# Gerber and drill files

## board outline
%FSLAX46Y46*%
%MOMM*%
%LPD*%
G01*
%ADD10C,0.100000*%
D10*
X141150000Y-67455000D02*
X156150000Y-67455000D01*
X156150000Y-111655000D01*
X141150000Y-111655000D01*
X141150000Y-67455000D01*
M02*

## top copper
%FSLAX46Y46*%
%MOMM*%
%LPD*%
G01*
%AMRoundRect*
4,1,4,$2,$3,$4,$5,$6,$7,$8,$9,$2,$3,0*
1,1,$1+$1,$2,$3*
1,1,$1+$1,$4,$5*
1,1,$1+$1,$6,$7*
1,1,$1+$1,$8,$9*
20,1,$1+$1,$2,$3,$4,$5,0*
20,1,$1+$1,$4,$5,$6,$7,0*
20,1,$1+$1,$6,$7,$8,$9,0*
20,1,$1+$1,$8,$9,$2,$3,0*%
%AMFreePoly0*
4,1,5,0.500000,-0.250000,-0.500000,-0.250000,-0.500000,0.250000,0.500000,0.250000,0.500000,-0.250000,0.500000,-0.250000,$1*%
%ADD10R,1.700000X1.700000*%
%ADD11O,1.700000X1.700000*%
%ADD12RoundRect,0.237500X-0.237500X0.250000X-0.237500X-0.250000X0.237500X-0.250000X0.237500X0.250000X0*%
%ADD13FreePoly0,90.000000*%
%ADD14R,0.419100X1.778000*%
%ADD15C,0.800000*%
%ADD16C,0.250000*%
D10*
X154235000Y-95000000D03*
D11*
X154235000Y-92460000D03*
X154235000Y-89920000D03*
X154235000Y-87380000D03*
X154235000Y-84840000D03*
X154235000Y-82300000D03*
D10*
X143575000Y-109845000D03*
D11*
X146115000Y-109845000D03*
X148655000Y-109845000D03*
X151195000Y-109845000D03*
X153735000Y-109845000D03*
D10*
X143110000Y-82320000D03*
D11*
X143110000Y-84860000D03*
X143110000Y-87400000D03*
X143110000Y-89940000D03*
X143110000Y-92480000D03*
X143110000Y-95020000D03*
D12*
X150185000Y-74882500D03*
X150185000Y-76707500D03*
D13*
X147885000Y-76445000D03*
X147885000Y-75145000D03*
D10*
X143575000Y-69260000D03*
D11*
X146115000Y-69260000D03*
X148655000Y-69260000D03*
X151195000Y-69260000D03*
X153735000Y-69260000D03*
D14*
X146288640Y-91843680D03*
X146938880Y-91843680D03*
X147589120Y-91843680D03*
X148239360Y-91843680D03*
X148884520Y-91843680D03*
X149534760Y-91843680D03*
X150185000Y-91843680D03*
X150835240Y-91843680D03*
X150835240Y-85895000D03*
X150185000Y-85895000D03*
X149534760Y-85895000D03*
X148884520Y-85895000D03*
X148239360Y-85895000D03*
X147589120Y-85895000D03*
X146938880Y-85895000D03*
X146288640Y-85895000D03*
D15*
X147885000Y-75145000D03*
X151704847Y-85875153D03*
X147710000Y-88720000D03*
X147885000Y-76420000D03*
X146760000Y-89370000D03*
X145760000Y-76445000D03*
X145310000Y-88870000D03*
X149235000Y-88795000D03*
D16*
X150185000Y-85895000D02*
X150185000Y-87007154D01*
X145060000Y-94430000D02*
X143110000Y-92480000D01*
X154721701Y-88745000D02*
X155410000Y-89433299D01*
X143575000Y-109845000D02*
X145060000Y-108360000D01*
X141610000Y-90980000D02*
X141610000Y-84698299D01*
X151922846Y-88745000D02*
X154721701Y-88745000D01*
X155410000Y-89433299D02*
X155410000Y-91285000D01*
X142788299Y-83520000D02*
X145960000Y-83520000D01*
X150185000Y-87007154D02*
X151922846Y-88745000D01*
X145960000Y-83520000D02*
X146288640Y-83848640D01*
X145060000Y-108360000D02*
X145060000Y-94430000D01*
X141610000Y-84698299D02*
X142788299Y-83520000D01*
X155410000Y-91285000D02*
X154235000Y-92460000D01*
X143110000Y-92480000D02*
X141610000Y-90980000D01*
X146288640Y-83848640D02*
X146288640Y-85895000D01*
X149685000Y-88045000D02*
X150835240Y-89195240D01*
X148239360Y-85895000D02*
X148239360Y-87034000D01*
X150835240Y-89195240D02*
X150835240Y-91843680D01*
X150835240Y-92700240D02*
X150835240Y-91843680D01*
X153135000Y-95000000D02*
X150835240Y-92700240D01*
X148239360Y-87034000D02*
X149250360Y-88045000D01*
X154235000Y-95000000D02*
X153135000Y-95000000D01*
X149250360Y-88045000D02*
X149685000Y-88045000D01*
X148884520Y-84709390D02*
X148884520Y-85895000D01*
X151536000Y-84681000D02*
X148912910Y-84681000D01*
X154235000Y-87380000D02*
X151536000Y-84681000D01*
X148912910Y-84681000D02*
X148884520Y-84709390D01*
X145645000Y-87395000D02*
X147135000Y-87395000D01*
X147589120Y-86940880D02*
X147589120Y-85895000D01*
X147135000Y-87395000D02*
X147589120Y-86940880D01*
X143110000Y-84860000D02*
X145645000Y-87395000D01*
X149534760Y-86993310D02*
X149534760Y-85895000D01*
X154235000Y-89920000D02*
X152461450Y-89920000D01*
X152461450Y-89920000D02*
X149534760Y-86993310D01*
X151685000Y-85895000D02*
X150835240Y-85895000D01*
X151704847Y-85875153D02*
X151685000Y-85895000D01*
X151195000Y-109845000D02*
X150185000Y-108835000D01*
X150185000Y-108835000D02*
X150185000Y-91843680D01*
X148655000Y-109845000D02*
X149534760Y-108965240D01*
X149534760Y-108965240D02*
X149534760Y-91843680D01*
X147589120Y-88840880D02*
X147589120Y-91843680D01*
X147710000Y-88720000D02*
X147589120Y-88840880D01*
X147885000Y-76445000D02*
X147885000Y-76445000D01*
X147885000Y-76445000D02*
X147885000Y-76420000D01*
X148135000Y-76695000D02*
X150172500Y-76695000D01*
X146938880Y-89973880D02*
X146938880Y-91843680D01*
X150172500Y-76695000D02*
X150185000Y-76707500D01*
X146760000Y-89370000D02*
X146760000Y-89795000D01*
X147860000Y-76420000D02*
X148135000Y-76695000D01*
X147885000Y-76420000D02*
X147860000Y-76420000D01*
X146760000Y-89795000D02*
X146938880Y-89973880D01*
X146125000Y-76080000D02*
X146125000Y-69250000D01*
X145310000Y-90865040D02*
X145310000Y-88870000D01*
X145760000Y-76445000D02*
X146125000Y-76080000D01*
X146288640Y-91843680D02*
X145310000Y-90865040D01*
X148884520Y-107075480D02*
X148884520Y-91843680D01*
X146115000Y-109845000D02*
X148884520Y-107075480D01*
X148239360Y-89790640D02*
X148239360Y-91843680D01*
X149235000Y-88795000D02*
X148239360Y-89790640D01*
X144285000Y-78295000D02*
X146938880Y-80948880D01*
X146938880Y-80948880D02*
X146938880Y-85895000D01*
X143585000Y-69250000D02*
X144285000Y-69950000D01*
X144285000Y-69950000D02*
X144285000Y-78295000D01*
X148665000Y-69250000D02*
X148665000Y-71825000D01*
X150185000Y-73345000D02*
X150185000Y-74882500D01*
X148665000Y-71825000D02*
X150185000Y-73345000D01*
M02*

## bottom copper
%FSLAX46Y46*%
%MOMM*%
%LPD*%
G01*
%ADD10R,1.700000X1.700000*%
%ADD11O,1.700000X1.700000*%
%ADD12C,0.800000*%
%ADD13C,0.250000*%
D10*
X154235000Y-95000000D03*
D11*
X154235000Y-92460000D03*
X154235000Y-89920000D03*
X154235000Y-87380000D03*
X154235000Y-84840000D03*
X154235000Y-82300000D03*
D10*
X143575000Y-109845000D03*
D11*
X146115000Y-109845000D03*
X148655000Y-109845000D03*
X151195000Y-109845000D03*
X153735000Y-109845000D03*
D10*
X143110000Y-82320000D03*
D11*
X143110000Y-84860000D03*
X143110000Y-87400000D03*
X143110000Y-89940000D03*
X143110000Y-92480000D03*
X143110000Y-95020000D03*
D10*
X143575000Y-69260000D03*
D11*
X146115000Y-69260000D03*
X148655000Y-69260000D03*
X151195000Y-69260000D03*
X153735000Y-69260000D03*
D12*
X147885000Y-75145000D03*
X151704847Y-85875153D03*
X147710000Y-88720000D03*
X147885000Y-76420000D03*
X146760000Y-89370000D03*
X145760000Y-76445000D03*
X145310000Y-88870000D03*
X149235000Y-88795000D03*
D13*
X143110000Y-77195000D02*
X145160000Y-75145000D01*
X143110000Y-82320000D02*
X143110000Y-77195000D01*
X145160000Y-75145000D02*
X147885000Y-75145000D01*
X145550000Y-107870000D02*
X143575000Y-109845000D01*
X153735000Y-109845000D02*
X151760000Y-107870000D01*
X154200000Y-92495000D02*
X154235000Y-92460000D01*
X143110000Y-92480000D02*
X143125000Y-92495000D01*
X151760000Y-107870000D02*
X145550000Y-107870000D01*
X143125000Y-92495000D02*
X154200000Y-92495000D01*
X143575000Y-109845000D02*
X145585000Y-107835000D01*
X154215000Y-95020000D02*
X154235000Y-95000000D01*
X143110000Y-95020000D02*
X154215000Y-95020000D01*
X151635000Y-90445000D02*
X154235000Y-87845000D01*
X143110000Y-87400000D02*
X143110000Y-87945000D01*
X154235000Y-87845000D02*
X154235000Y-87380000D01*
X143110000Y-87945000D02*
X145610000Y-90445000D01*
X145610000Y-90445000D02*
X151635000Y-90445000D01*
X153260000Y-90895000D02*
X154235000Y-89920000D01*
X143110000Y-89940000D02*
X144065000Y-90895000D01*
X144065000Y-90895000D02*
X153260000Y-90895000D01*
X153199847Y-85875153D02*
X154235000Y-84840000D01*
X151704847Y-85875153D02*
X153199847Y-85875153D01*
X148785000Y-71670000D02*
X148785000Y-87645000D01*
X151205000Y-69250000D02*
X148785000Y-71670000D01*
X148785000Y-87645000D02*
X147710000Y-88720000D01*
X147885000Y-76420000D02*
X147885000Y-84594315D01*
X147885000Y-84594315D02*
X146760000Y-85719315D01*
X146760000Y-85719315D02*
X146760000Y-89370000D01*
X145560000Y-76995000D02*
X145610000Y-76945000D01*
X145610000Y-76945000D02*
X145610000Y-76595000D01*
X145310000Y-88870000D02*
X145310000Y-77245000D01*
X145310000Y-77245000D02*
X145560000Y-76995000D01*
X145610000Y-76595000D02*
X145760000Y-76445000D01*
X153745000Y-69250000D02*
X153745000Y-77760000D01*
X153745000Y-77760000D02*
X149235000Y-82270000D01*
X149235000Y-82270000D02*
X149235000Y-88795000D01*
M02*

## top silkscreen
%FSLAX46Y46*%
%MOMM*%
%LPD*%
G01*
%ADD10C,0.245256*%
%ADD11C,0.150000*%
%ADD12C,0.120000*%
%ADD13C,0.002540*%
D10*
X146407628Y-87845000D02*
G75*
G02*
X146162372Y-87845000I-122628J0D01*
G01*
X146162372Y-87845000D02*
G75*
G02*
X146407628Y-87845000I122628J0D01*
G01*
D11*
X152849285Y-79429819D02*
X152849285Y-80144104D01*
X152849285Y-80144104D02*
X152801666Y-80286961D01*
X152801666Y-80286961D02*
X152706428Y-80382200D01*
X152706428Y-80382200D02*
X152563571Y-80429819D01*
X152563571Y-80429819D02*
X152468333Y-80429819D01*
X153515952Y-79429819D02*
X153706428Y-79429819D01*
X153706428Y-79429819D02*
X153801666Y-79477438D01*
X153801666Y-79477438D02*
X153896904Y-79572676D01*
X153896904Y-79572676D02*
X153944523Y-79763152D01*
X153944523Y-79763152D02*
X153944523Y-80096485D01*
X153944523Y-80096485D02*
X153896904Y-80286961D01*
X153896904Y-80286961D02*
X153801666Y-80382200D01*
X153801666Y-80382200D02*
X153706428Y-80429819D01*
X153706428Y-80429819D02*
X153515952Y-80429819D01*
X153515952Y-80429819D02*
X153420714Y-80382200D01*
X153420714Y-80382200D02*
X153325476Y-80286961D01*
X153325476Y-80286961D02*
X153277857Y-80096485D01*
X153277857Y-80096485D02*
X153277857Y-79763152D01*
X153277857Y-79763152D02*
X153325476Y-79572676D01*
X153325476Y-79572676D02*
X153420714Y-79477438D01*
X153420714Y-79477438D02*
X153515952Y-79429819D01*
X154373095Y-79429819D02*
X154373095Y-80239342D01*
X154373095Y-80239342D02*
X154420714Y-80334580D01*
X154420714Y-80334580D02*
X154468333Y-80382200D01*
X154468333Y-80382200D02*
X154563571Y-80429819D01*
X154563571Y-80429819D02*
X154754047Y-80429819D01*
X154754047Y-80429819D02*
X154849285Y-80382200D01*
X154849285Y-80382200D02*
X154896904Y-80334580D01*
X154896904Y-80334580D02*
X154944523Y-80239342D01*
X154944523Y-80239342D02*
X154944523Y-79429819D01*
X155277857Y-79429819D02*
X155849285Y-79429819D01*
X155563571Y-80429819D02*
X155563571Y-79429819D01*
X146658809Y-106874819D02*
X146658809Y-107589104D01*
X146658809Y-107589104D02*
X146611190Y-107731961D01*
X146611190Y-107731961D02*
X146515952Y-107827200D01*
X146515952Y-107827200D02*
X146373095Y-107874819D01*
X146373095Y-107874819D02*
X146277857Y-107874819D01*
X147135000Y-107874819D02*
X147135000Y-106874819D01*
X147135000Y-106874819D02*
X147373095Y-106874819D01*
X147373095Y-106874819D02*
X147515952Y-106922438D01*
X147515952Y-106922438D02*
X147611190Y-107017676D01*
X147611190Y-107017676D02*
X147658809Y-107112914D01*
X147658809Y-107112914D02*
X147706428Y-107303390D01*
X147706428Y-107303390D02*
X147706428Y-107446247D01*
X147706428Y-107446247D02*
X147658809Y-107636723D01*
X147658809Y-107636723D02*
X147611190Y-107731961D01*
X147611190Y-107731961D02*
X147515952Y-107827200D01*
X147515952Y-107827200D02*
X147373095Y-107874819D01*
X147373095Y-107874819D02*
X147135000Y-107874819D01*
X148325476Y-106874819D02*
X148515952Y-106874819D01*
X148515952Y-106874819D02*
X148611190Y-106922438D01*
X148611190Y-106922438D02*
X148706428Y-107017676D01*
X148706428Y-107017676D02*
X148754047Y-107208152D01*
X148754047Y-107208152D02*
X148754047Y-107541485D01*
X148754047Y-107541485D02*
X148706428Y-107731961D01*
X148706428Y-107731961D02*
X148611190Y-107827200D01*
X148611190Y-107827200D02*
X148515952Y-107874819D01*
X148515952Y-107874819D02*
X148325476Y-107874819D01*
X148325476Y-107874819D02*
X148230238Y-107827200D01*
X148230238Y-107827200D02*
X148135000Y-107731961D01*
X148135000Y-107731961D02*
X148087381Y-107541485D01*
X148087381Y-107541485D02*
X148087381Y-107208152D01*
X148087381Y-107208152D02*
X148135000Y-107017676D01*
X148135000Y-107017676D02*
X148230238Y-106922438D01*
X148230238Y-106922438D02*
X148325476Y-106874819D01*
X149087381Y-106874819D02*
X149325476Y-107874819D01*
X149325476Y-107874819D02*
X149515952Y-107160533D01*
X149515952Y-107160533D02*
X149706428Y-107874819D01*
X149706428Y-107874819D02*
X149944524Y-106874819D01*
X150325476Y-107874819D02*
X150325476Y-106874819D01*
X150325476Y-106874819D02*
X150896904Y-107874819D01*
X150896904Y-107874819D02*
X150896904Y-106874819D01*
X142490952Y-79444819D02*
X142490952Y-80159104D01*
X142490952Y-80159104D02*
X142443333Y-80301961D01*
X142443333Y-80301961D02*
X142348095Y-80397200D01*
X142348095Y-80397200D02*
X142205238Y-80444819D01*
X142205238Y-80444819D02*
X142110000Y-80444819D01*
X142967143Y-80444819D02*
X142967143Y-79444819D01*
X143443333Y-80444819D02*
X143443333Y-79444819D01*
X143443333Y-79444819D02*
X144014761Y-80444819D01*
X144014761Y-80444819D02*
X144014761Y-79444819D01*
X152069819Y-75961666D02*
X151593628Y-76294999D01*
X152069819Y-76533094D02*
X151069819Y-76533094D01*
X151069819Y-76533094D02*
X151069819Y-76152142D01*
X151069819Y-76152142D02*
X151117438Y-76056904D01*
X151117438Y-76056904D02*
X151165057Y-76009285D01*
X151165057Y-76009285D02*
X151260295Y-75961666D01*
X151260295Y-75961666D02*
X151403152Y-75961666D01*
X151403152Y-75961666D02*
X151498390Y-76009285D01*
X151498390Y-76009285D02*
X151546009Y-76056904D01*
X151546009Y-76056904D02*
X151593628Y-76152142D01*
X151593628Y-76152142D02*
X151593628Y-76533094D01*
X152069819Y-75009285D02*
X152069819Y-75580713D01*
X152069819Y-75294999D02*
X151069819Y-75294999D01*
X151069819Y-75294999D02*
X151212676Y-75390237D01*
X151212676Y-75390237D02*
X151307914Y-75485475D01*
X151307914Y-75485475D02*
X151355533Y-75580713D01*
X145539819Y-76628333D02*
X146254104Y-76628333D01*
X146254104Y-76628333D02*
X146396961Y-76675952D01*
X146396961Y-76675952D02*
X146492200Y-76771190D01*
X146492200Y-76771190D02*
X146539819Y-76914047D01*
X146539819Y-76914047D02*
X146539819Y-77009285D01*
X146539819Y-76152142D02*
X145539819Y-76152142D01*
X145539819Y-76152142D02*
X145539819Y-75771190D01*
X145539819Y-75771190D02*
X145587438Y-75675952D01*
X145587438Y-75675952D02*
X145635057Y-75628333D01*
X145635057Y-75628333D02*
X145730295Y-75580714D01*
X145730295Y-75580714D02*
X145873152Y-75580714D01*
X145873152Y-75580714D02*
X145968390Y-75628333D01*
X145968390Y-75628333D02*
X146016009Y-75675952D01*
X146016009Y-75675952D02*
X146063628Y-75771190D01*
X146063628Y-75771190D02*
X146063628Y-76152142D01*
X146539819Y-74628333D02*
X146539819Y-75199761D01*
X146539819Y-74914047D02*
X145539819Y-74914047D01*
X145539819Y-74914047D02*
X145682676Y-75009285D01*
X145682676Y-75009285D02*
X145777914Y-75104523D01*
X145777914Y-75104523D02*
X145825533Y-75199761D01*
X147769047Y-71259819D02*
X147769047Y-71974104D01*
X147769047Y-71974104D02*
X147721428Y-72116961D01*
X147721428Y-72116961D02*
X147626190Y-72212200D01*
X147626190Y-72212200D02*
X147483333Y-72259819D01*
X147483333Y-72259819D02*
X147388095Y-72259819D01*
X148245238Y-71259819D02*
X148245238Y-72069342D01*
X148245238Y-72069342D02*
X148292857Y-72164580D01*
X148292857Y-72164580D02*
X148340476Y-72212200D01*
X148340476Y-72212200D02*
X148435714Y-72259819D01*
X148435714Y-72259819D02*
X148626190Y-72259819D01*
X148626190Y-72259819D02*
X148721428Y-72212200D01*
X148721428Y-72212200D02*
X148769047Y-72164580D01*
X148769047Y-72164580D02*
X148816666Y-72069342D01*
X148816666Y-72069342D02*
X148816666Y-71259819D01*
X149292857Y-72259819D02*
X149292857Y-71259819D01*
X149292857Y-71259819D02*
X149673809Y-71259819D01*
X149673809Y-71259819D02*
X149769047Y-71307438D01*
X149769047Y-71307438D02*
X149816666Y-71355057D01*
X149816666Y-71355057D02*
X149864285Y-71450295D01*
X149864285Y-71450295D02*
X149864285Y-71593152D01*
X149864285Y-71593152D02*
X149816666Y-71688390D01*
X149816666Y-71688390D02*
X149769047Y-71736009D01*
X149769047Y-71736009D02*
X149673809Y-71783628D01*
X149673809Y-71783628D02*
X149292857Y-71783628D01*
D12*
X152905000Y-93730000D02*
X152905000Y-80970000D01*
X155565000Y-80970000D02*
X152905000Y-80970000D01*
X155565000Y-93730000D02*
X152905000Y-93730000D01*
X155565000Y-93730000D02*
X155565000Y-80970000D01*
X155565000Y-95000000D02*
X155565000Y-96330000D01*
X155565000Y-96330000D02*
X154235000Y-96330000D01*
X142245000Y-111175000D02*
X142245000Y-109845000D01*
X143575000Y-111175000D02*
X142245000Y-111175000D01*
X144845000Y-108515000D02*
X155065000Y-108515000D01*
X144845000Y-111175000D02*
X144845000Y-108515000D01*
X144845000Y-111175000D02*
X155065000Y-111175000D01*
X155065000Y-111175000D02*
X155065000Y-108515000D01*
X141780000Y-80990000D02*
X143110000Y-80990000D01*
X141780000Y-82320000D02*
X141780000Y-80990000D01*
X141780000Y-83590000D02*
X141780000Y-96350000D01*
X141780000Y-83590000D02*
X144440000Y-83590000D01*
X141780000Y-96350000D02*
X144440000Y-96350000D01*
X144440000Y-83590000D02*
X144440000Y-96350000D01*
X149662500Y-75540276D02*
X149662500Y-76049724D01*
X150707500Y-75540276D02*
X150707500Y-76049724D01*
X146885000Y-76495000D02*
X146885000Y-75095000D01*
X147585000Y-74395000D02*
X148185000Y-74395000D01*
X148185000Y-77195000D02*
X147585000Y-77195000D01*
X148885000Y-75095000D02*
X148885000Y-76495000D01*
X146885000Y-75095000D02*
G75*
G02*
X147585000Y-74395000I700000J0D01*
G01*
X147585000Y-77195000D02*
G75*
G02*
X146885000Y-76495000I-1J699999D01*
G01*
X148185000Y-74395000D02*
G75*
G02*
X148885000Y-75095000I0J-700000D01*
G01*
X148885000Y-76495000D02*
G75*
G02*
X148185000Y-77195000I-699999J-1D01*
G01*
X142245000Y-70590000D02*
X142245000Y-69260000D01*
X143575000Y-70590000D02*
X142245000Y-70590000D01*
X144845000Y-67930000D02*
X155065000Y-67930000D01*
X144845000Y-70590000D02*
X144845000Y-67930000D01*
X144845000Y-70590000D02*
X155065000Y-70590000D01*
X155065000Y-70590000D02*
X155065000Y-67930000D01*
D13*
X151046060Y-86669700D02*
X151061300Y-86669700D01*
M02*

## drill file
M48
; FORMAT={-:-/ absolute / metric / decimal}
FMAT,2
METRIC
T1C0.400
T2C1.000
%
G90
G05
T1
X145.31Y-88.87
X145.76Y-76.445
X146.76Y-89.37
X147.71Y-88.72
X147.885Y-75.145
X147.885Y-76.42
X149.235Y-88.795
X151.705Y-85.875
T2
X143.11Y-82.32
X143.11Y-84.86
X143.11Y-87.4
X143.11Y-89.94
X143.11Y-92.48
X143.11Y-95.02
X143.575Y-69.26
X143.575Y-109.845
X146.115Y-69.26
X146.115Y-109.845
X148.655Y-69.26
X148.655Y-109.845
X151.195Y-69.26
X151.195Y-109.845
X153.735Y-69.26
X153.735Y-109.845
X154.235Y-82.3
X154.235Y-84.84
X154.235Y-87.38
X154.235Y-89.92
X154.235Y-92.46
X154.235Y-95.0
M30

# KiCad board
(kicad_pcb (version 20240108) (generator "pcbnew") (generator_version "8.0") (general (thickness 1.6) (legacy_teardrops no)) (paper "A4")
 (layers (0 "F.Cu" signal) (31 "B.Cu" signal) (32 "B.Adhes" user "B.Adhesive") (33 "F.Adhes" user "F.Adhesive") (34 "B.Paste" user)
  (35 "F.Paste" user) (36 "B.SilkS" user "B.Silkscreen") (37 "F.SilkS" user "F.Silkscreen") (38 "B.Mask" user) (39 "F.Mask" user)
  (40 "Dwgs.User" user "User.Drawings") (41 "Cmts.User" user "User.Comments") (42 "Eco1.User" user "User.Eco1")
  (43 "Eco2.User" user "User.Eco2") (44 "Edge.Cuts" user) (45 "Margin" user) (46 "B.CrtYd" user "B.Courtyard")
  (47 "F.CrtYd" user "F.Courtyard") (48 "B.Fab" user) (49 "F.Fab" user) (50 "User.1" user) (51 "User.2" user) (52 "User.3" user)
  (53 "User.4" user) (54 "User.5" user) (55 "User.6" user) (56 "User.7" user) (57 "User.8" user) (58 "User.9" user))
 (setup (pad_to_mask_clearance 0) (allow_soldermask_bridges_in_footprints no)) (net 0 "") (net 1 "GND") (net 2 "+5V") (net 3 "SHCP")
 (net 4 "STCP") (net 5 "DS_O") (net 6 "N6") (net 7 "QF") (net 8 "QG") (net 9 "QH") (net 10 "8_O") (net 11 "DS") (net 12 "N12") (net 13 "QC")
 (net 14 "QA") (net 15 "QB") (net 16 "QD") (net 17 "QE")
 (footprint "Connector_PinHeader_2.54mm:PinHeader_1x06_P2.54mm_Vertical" (layer "F.Cu") (at 154.235 95 180)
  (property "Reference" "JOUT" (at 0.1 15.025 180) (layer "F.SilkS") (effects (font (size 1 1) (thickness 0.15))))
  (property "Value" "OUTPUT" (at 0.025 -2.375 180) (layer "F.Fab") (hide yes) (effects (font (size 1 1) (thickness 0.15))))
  (fp_line (start 1.33 1.27) (end 1.33 14.03) (stroke (width 0.12) (type solid)) (layer "F.SilkS"))
  (fp_line (start -1.33 14.03) (end 1.33 14.03) (stroke (width 0.12) (type solid)) (layer "F.SilkS"))
  (fp_line (start -1.33 1.27) (end 1.33 1.27) (stroke (width 0.12) (type solid)) (layer "F.SilkS"))
  (fp_line (start -1.33 1.27) (end -1.33 14.03) (stroke (width 0.12) (type solid)) (layer "F.SilkS"))
  (fp_line (start -1.33 0) (end -1.33 -1.33) (stroke (width 0.12) (type solid)) (layer "F.SilkS"))
  (fp_line (start -1.33 -1.33) (end 0 -1.33) (stroke (width 0.12) (type solid)) (layer "F.SilkS"))
  (pad "1" thru_hole rect (at 0 0 180) (size 1.7 1.7) (drill 1) (layers "*.Cu" "*.Mask") (remove_unused_layers no) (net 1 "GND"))
  (pad "2" thru_hole oval (at 0 2.54 180) (size 1.7 1.7) (drill 1) (layers "*.Cu" "*.Mask") (remove_unused_layers no) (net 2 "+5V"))
  (pad "3" thru_hole oval (at 0 5.08 180) (size 1.7 1.7) (drill 1) (layers "*.Cu" "*.Mask") (remove_unused_layers no) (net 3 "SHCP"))
  (pad "4" thru_hole oval (at 0 7.62 180) (size 1.7 1.7) (drill 1) (layers "*.Cu" "*.Mask") (remove_unused_layers no) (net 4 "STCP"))
  (pad "5" thru_hole oval (at 0 10.16 180) (size 1.7 1.7) (drill 1) (layers "*.Cu" "*.Mask") (remove_unused_layers no) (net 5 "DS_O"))
  (pad "6" thru_hole oval (at 0 12.7 180) (size 1.7 1.7) (drill 1) (layers "*.Cu" "*.Mask") (remove_unused_layers no) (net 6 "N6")))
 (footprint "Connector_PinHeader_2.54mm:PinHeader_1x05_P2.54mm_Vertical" (layer "F.Cu") (at 143.575 109.845 90)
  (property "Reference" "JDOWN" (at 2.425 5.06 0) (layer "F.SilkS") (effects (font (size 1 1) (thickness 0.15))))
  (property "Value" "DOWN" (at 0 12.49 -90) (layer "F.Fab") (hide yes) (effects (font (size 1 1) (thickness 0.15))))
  (fp_line (start -1.33 -1.33) (end 0 -1.33) (stroke (width 0.12) (type solid)) (layer "F.SilkS"))
  (fp_line (start -1.33 0) (end -1.33 -1.33) (stroke (width 0.12) (type solid)) (layer "F.SilkS"))
  (fp_line (start 1.33 1.27) (end 1.33 11.49) (stroke (width 0.12) (type solid)) (layer "F.SilkS"))
  (fp_line (start -1.33 1.27) (end 1.33 1.27) (stroke (width 0.12) (type solid)) (layer "F.SilkS"))
  (fp_line (start -1.33 1.27) (end -1.33 11.49) (stroke (width 0.12) (type solid)) (layer "F.SilkS"))
  (fp_line (start -1.33 11.49) (end 1.33 11.49) (stroke (width 0.12) (type solid)) (layer "F.SilkS"))
  (pad "1" thru_hole rect (at 0 0 90) (size 1.7 1.7) (drill 1) (layers "*.Cu" "*.Mask") (remove_unused_layers no) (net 2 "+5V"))
  (pad "2" thru_hole oval (at 0 2.54 90) (size 1.7 1.7) (drill 1) (layers "*.Cu" "*.Mask") (remove_unused_layers no) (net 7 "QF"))
  (pad "3" thru_hole oval (at 0 5.08 90) (size 1.7 1.7) (drill 1) (layers "*.Cu" "*.Mask") (remove_unused_layers no) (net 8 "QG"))
  (pad "4" thru_hole oval (at 0 7.62 90) (size 1.7 1.7) (drill 1) (layers "*.Cu" "*.Mask") (remove_unused_layers no) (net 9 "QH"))
  (pad "5" thru_hole oval (at 0 10.16 90) (size 1.7 1.7) (drill 1) (layers "*.Cu" "*.Mask") (remove_unused_layers no) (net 2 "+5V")))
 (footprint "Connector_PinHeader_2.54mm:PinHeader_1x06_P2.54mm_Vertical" (layer "F.Cu") (at 143.11 82.32)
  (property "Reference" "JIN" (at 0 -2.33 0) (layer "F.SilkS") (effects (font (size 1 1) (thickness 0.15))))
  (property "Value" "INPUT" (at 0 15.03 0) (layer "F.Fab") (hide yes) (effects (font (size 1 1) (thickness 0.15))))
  (fp_line (start -1.33 -1.33) (end 0 -1.33) (stroke (width 0.12) (type solid)) (layer "F.SilkS"))
  (fp_line (start -1.33 0) (end -1.33 -1.33) (stroke (width 0.12) (type solid)) (layer "F.SilkS"))
  (fp_line (start -1.33 1.27) (end -1.33 14.03) (stroke (width 0.12) (type solid)) (layer "F.SilkS"))
  (fp_line (start -1.33 1.27) (end 1.33 1.27) (stroke (width 0.12) (type solid)) (layer "F.SilkS"))
  (fp_line (start -1.33 14.03) (end 1.33 14.03) (stroke (width 0.12) (type solid)) (layer "F.SilkS"))
  (fp_line (start 1.33 1.27) (end 1.33 14.03) (stroke (width 0.12) (type solid)) (layer "F.SilkS"))
  (pad "1" thru_hole rect (at 0 0) (size 1.7 1.7) (drill 1) (layers "*.Cu" "*.Mask") (remove_unused_layers no) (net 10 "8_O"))
  (pad "2" thru_hole oval (at 0 2.54) (size 1.7 1.7) (drill 1) (layers "*.Cu" "*.Mask") (remove_unused_layers no) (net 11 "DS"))
  (pad "3" thru_hole oval (at 0 5.08) (size 1.7 1.7) (drill 1) (layers "*.Cu" "*.Mask") (remove_unused_layers no) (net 4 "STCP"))
  (pad "4" thru_hole oval (at 0 7.62) (size 1.7 1.7) (drill 1) (layers "*.Cu" "*.Mask") (remove_unused_layers no) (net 3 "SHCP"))
  (pad "5" thru_hole oval (at 0 10.16) (size 1.7 1.7) (drill 1) (layers "*.Cu" "*.Mask") (remove_unused_layers no) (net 2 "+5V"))
  (pad "6" thru_hole oval (at 0 12.7) (size 1.7 1.7) (drill 1) (layers "*.Cu" "*.Mask") (remove_unused_layers no) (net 1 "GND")))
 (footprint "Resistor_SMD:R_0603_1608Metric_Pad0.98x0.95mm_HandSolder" (layer "F.Cu") (at 150.185 75.795 -90)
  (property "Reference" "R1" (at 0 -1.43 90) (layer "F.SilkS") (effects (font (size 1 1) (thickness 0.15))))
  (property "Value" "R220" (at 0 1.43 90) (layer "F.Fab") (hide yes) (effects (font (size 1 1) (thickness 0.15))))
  (fp_line (start -0.254724 0.5225) (end 0.254724 0.5225) (stroke (width 0.12) (type solid)) (layer "F.SilkS"))
  (fp_line (start -0.254724 -0.5225) (end 0.254724 -0.5225) (stroke (width 0.12) (type solid)) (layer "F.SilkS"))
  (pad "1" smd roundrect (at -0.9125 0 270) (size 0.975 0.95) (layers "F.Cu" "F.Paste" "F.Mask") (roundrect_rratio 0.25) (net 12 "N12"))
  (pad "2" smd roundrect (at 0.9125 0 270) (size 0.975 0.95) (layers "F.Cu" "F.Paste" "F.Mask") (roundrect_rratio 0.25) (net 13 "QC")))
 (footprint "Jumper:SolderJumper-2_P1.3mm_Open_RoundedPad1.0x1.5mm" (layer "F.Cu") (at 147.885 75.795 90)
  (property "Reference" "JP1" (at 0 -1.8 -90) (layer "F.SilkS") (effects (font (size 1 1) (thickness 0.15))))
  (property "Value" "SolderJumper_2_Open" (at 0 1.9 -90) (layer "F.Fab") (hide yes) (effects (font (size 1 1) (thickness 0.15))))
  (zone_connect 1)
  (fp_line (start -0.7 -1) (end 0.7 -1) (stroke (width 0.12) (type solid)) (layer "F.SilkS"))
  (fp_line (start 1.4 -0.3) (end 1.4 0.3) (stroke (width 0.12) (type solid)) (layer "F.SilkS"))
  (fp_line (start -1.4 0.3) (end -1.4 -0.3) (stroke (width 0.12) (type solid)) (layer "F.SilkS"))
  (fp_line (start 0.7 1) (end -0.7 1) (stroke (width 0.12) (type solid)) (layer "F.SilkS"))
  (fp_arc (start 0.7 -1) (mid 1.194975 -0.794975) (end 1.4 -0.3) (stroke (width 0.12) (type solid)) (layer "F.SilkS"))
  (fp_arc (start -1.4 -0.3) (mid -1.194975 -0.794975) (end -0.7 -1) (stroke (width 0.12) (type solid)) (layer "F.SilkS"))
  (fp_arc (start 1.4 0.3) (mid 1.194975 0.794975) (end 0.7 1) (stroke (width 0.12) (type solid)) (layer "F.SilkS"))
  (fp_arc (start -0.7 1) (mid -1.194975 0.794975) (end -1.4 0.3) (stroke (width 0.12) (type solid)) (layer "F.SilkS"))
  (pad "1" smd custom (at -0.65 0 90) (size 1 0.5) (layers "F.Cu" "F.Mask") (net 13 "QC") (zone_connect 2) (thermal_bridge_angle 45)
   (options (clearance outline) (anchor rect)) (primitives))
  (pad "2" smd custom (at 0.65 0 90) (size 1 0.5) (layers "F.Cu" "F.Mask") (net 10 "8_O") (zone_connect 2) (thermal_bridge_angle 45)
   (options (clearance outline) (anchor rect)) (primitives)))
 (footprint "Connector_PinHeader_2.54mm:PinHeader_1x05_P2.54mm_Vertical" (layer "F.Cu") (at 143.575 69.26 90)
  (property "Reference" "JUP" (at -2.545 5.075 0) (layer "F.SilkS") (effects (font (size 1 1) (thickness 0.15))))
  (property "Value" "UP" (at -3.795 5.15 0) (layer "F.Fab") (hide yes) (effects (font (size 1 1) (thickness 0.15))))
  (fp_line (start -1.33 -1.33) (end 0 -1.33) (stroke (width 0.12) (type solid)) (layer "F.SilkS"))
  (fp_line (start -1.33 0) (end -1.33 -1.33) (stroke (width 0.12) (type solid)) (layer "F.SilkS"))
  (fp_line (start 1.33 1.27) (end 1.33 11.49) (stroke (width 0.12) (type solid)) (layer "F.SilkS"))
  (fp_line (start -1.33 1.27) (end 1.33 1.27) (stroke (width 0.12) (type solid)) (layer "F.SilkS"))
  (fp_line (start -1.33 1.27) (end -1.33 11.49) (stroke (width 0.12) (type solid)) (layer "F.SilkS"))
  (fp_line (start -1.33 11.49) (end 1.33 11.49) (stroke (width 0.12) (type solid)) (layer "F.SilkS"))
  (pad "1" thru_hole rect (at 0 0 90) (size 1.7 1.7) (drill 1) (layers "*.Cu" "*.Mask") (remove_unused_layers no) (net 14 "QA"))
  (pad "2" thru_hole oval (at 0 2.54 90) (size 1.7 1.7) (drill 1) (layers "*.Cu" "*.Mask") (remove_unused_layers no) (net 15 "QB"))
  (pad "3" thru_hole oval (at 0 5.08 90) (size 1.7 1.7) (drill 1) (layers "*.Cu" "*.Mask") (remove_unused_layers no) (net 12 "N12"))
  (pad "4" thru_hole oval (at 0 7.62 90) (size 1.7 1.7) (drill 1) (layers "*.Cu" "*.Mask") (remove_unused_layers no) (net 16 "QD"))
  (pad "5" thru_hole oval (at 0 10.16 90) (size 1.7 1.7) (drill 1) (layers "*.Cu" "*.Mask") (remove_unused_layers no) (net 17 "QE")))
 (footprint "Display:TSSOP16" (layer "F.Cu") (at 148.56194 88.86934)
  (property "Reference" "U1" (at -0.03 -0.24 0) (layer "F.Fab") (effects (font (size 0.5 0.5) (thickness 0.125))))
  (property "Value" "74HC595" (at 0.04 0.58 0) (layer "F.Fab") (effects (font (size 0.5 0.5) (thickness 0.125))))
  (fp_line (start 2.48412 -2.19964) (end 2.49936 -2.19964) (stroke (width 0.00254) (type solid)) (layer "F.SilkS"))
  (pad "1" smd rect (at -2.2733 2.97434 180) (size 0.4191 1.778) (layers "F.Cu" "F.Paste" "F.Mask") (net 15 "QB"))
  (pad "2" smd rect (at -1.62306 2.97434 180) (size 0.4191 1.778) (layers "F.Cu" "F.Paste" "F.Mask") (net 13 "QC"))
  (pad "3" smd rect (at -0.97282 2.97434 180) (size 0.4191 1.778) (layers "F.Cu" "F.Paste" "F.Mask") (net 16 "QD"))
  (pad "4" smd rect (at -0.32258 2.97434 180) (size 0.4191 1.778) (layers "F.Cu" "F.Paste" "F.Mask") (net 17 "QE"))
  (pad "5" smd rect (at 0.32258 2.97434 180) (size 0.4191 1.778) (layers "F.Cu" "F.Paste" "F.Mask") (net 7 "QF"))
  (pad "6" smd rect (at 0.97282 2.97434 180) (size 0.4191 1.778) (layers "F.Cu" "F.Paste" "F.Mask") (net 8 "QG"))
  (pad "7" smd rect (at 1.62306 2.97434 180) (size 0.4191 1.778) (layers "F.Cu" "F.Paste" "F.Mask") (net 9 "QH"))
  (pad "8" smd rect (at 2.2733 2.97434 180) (size 0.4191 1.778) (layers "F.Cu" "F.Paste" "F.Mask") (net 1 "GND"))
  (pad "9" smd rect (at 2.2733 -2.97434) (size 0.4191 1.778) (layers "F.Cu" "F.Paste" "F.Mask") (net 5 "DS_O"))
  (pad "10" smd rect (at 1.62306 -2.97434) (size 0.4191 1.778) (layers "F.Cu" "F.Paste" "F.Mask") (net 2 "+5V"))
  (pad "11" smd rect (at 0.97282 -2.97434) (size 0.4191 1.778) (layers "F.Cu" "F.Paste" "F.Mask") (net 3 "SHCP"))
  (pad "12" smd rect (at 0.32258 -2.97434) (size 0.4191 1.778) (layers "F.Cu" "F.Paste" "F.Mask") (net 4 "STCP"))
  (pad "13" smd rect (at -0.32258 -2.97434) (size 0.4191 1.778) (layers "F.Cu" "F.Paste" "F.Mask") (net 1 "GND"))
  (pad "14" smd rect (at -0.97282 -2.97434) (size 0.4191 1.778) (layers "F.Cu" "F.Paste" "F.Mask") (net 11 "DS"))
  (pad "15" smd rect (at -1.62306 -2.97434) (size 0.4191 1.778) (layers "F.Cu" "F.Paste" "F.Mask") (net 14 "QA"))
  (pad "16" smd rect (at -2.2733 -2.97434) (size 0.4191 1.778) (layers "F.Cu" "F.Paste" "F.Mask") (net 2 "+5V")))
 (gr_circle (center 146.285 87.845) (end 146.480256 87.845) (stroke (width 0.1) (type solid)) (fill solid) (layer "F.SilkS"))
 (gr_rect (start 141.15 67.455) (end 156.15 111.655) (stroke (width 0.1) (type default)) (fill none) (layer "Edge.Cuts"))
 (via (at 147.885 75.145) (size 0.8) (drill 0.4) (layers "F.Cu" "B.Cu") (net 10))
 (segment (start 143.11 77.195) (end 145.16 75.145) (width 0.25) (layer "B.Cu") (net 10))
 (segment (start 143.11 82.32) (end 143.11 77.195) (width 0.25) (layer "B.Cu") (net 10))
 (segment (start 145.16 75.145) (end 147.885 75.145) (width 0.25) (layer "B.Cu") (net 10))
 (segment (start 150.185 85.895) (end 150.185 87.007154) (width 0.25) (layer "F.Cu") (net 2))
 (segment (start 145.06 94.43) (end 143.11 92.48) (width 0.25) (layer "F.Cu") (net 2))
 (segment (start 154.721701 88.745) (end 155.41 89.433299) (width 0.25) (layer "F.Cu") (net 2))
 (segment (start 143.575 109.845) (end 145.06 108.36) (width 0.25) (layer "F.Cu") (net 2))
 (segment (start 141.61 90.98) (end 141.61 84.698299) (width 0.25) (layer "F.Cu") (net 2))
 (segment (start 151.922846 88.745) (end 154.721701 88.745) (width 0.25) (layer "F.Cu") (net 2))
 (segment (start 155.41 89.433299) (end 155.41 91.285) (width 0.25) (layer "F.Cu") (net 2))
 (segment (start 142.788299 83.52) (end 145.96 83.52) (width 0.25) (layer "F.Cu") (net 2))
 (segment (start 150.185 87.007154) (end 151.922846 88.745) (width 0.25) (layer "F.Cu") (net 2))
 (segment (start 145.96 83.52) (end 146.28864 83.84864) (width 0.25) (layer "F.Cu") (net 2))
 (segment (start 145.06 108.36) (end 145.06 94.43) (width 0.25) (layer "F.Cu") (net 2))
 (segment (start 141.61 84.698299) (end 142.788299 83.52) (width 0.25) (layer "F.Cu") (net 2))
 (segment (start 155.41 91.285) (end 154.235 92.46) (width 0.25) (layer "F.Cu") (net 2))
 (segment (start 143.11 92.48) (end 141.61 90.98) (width 0.25) (layer "F.Cu") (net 2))
 (segment (start 146.28864 83.84864) (end 146.28864 85.895) (width 0.25) (layer "F.Cu") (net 2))
 (segment (start 145.55 107.87) (end 143.575 109.845) (width 0.25) (layer "B.Cu") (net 2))
 (segment (start 153.735 109.845) (end 151.76 107.87) (width 0.25) (layer "B.Cu") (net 2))
 (segment (start 154.2 92.495) (end 154.235 92.46) (width 0.25) (layer "B.Cu") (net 2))
 (segment (start 143.11 92.48) (end 143.125 92.495) (width 0.25) (layer "B.Cu") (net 2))
 (segment (start 151.76 107.87) (end 145.55 107.87) (width 0.25) (layer "B.Cu") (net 2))
 (segment (start 143.125 92.495) (end 154.2 92.495) (width 0.25) (layer "B.Cu") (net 2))
 (segment (start 143.575 109.845) (end 145.585 107.835) (width 0.25) (layer "B.Cu") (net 2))
 (segment (start 149.685 88.045) (end 150.83524 89.19524) (width 0.25) (layer "F.Cu") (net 1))
 (segment (start 148.23936 85.895) (end 148.23936 87.034) (width 0.25) (layer "F.Cu") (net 1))
 (segment (start 150.83524 89.19524) (end 150.83524 91.84368) (width 0.25) (layer "F.Cu") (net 1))
 (segment (start 150.83524 92.70024) (end 150.83524 91.84368) (width 0.25) (layer "F.Cu") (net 1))
 (segment (start 153.135 95) (end 150.83524 92.70024) (width 0.25) (layer "F.Cu") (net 1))
 (segment (start 148.23936 87.034) (end 149.25036 88.045) (width 0.25) (layer "F.Cu") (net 1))
 (segment (start 154.235 95) (end 153.135 95) (width 0.25) (layer "F.Cu") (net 1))
 (segment (start 149.25036 88.045) (end 149.685 88.045) (width 0.25) (layer "F.Cu") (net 1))
 (segment (start 154.215 95.02) (end 154.235 95) (width 0.25) (layer "B.Cu") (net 1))
 (segment (start 143.11 95.02) (end 154.215 95.02) (width 0.25) (layer "B.Cu") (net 1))
 (segment (start 148.88452 84.70939) (end 148.88452 85.895) (width 0.25) (layer "F.Cu") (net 4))
 (segment (start 151.536 84.681) (end 148.91291 84.681) (width 0.25) (layer "F.Cu") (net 4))
 (segment (start 154.235 87.38) (end 151.536 84.681) (width 0.25) (layer "F.Cu") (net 4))
 (segment (start 148.91291 84.681) (end 148.88452 84.70939) (width 0.25) (layer "F.Cu") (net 4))
 (segment (start 151.635 90.445) (end 154.235 87.845) (width 0.25) (layer "B.Cu") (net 4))
 (segment (start 143.11 87.4) (end 143.11 87.945) (width 0.25) (layer "B.Cu") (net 4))
 (segment (start 154.235 87.845) (end 154.235 87.38) (width 0.25) (layer "B.Cu") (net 4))
 (segment (start 143.11 87.945) (end 145.61 90.445) (width 0.25) (layer "B.Cu") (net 4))
 (segment (start 145.61 90.445) (end 151.635 90.445) (width 0.25) (layer "B.Cu") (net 4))
 (segment (start 145.645 87.395) (end 147.135 87.395) (width 0.25) (layer "F.Cu") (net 11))
 (segment (start 147.58912 86.94088) (end 147.58912 85.895) (width 0.25) (layer "F.Cu") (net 11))
 (segment (start 147.135 87.395) (end 147.58912 86.94088) (width 0.25) (layer "F.Cu") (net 11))
 (segment (start 143.11 84.86) (end 145.645 87.395) (width 0.25) (layer "F.Cu") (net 11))
 (segment (start 149.53476 86.99331) (end 149.53476 85.895) (width 0.25) (layer "F.Cu") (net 3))
 (segment (start 154.235 89.92) (end 152.46145 89.92) (width 0.25) (layer "F.Cu") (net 3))
 (segment (start 152.46145 89.92) (end 149.53476 86.99331) (width 0.25) (layer "F.Cu") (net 3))
 (segment (start 153.26 90.895) (end 154.235 89.92) (width 0.25) (layer "B.Cu") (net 3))
 (segment (start 143.11 89.94) (end 144.065 90.895) (width 0.25) (layer "B.Cu") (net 3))
 (segment (start 144.065 90.895) (end 153.26 90.895) (width 0.25) (layer "B.Cu") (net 3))
 (segment (start 151.685 85.895) (end 150.83524 85.895) (width 0.25) (layer "F.Cu") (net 5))
 (segment (start 151.704847 85.875153) (end 151.685 85.895) (width 0.25) (layer "F.Cu") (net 5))
 (via (at 151.704847 85.875153) (size 0.8) (drill 0.4) (layers "F.Cu" "B.Cu") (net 5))
 (segment (start 153.199847 85.875153) (end 154.235 84.84) (width 0.25) (layer "B.Cu") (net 5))
 (segment (start 151.704847 85.875153) (end 153.199847 85.875153) (width 0.25) (layer "B.Cu") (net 5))
 (segment (start 151.195 109.845) (end 150.185 108.835) (width 0.25) (layer "F.Cu") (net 9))
 (segment (start 150.185 108.835) (end 150.185 91.84368) (width 0.25) (layer "F.Cu") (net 9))
 (segment (start 148.655 109.845) (end 149.53476 108.96524) (width 0.25) (layer "F.Cu") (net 8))
 (segment (start 149.53476 108.96524) (end 149.53476 91.84368) (width 0.25) (layer "F.Cu") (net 8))
 (segment (start 147.58912 88.84088) (end 147.58912 91.84368) (width 0.25) (layer "F.Cu") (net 16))
 (segment (start 147.71 88.72) (end 147.58912 88.84088) (width 0.25) (layer "F.Cu") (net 16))
 (via (at 147.71 88.72) (size 0.8) (drill 0.4) (layers "F.Cu" "B.Cu") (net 16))
 (segment (start 148.785 71.67) (end 148.785 87.645) (width 0.25) (layer "B.Cu") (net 16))
 (segment (start 151.205 69.25) (end 148.785 71.67) (width 0.25) (layer "B.Cu") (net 16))
 (segment (start 148.785 87.645) (end 147.71 88.72) (width 0.25) (layer "B.Cu") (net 16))
 (segment (start 147.885 76.445) (end 147.885 76.445) (width 0.25) (layer "F.Cu") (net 13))
 (segment (start 147.885 76.445) (end 147.885 76.42) (width 0.25) (layer "F.Cu") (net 13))
 (segment (start 148.135 76.695) (end 150.1725 76.695) (width 0.25) (layer "F.Cu") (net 13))
 (segment (start 146.93888 89.97388) (end 146.93888 91.84368) (width 0.25) (layer "F.Cu") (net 13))
 (segment (start 150.1725 76.695) (end 150.185 76.7075) (width 0.25) (layer "F.Cu") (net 13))
 (segment (start 146.76 89.37) (end 146.76 89.795) (width 0.25) (layer "F.Cu") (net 13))
 (segment (start 147.86 76.42) (end 148.135 76.695) (width 0.25) (layer "F.Cu") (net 13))
 (segment (start 147.885 76.42) (end 147.86 76.42) (width 0.25) (layer "F.Cu") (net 13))
 (segment (start 146.76 89.795) (end 146.93888 89.97388) (width 0.25) (layer "F.Cu") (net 13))
 (via (at 147.885 76.42) (size 0.8) (drill 0.4) (layers "F.Cu" "B.Cu") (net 13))
 (via (at 146.76 89.37) (size 0.8) (drill 0.4) (layers "F.Cu" "B.Cu") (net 13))
 (segment (start 147.885 76.42) (end 147.885 84.594315) (width 0.25) (layer "B.Cu") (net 13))
 (segment (start 147.885 84.594315) (end 146.76 85.719315) (width 0.25) (layer "B.Cu") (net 13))
 (segment (start 146.76 85.719315) (end 146.76 89.37) (width 0.25) (layer "B.Cu") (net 13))
 (segment (start 146.125 76.08) (end 146.125 69.25) (width 0.25) (layer "F.Cu") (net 15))
 (segment (start 145.31 90.86504) (end 145.31 88.87) (width 0.25) (layer "F.Cu") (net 15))
 (segment (start 145.76 76.445) (end 146.125 76.08) (width 0.25) (layer "F.Cu") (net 15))
 (segment (start 146.28864 91.84368) (end 145.31 90.86504) (width 0.25) (layer "F.Cu") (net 15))
 (via (at 145.76 76.445) (size 0.8) (drill 0.4) (layers "F.Cu" "B.Cu") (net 15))
 (via (at 145.31 88.87) (size 0.8) (drill 0.4) (layers "F.Cu" "B.Cu") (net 15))
 (segment (start 145.56 76.995) (end 145.61 76.945) (width 0.25) (layer "B.Cu") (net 15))
 (segment (start 145.61 76.945) (end 145.61 76.595) (width 0.25) (layer "B.Cu") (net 15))
 (segment (start 145.31 88.87) (end 145.31 77.245) (width 0.25) (layer "B.Cu") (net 15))
 (segment (start 145.31 77.245) (end 145.56 76.995) (width 0.25) (layer "B.Cu") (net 15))
 (segment (start 145.61 76.595) (end 145.76 76.445) (width 0.25) (layer "B.Cu") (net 15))
 (segment (start 148.88452 107.07548) (end 148.88452 91.84368) (width 0.25) (layer "F.Cu") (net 7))
 (segment (start 146.115 109.845) (end 148.88452 107.07548) (width 0.25) (layer "F.Cu") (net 7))
 (segment (start 148.23936 89.79064) (end 148.23936 91.84368) (width 0.25) (layer "F.Cu") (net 17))
 (segment (start 149.235 88.795) (end 148.23936 89.79064) (width 0.25) (layer "F.Cu") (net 17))
 (via (at 149.235 88.795) (size 0.8) (drill 0.4) (layers "F.Cu" "B.Cu") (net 17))
 (segment (start 153.745 69.25) (end 153.745 77.76) (width 0.25) (layer "B.Cu") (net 17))
 (segment (start 153.745 77.76) (end 149.235 82.27) (width 0.25) (layer "B.Cu") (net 17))
 (segment (start 149.235 82.27) (end 149.235 88.795) (width 0.25) (layer "B.Cu") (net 17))
 (segment (start 144.285 78.295) (end 146.93888 80.94888) (width 0.25) (layer "F.Cu") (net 14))
 (segment (start 146.93888 80.94888) (end 146.93888 85.895) (width 0.25) (layer "F.Cu") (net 14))
 (segment (start 143.585 69.25) (end 144.285 69.95) (width 0.25) (layer "F.Cu") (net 14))
 (segment (start 144.285 69.95) (end 144.285 78.295) (width 0.25) (layer "F.Cu") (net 14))
 (segment (start 148.665 69.25) (end 148.665 71.825) (width 0.25) (layer "F.Cu") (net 12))
 (segment (start 150.185 73.345) (end 150.185 74.8825) (width 0.25) (layer "F.Cu") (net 12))
 (segment (start 148.665 71.825) (end 150.185 73.345) (width 0.25) (layer "F.Cu") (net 12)))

